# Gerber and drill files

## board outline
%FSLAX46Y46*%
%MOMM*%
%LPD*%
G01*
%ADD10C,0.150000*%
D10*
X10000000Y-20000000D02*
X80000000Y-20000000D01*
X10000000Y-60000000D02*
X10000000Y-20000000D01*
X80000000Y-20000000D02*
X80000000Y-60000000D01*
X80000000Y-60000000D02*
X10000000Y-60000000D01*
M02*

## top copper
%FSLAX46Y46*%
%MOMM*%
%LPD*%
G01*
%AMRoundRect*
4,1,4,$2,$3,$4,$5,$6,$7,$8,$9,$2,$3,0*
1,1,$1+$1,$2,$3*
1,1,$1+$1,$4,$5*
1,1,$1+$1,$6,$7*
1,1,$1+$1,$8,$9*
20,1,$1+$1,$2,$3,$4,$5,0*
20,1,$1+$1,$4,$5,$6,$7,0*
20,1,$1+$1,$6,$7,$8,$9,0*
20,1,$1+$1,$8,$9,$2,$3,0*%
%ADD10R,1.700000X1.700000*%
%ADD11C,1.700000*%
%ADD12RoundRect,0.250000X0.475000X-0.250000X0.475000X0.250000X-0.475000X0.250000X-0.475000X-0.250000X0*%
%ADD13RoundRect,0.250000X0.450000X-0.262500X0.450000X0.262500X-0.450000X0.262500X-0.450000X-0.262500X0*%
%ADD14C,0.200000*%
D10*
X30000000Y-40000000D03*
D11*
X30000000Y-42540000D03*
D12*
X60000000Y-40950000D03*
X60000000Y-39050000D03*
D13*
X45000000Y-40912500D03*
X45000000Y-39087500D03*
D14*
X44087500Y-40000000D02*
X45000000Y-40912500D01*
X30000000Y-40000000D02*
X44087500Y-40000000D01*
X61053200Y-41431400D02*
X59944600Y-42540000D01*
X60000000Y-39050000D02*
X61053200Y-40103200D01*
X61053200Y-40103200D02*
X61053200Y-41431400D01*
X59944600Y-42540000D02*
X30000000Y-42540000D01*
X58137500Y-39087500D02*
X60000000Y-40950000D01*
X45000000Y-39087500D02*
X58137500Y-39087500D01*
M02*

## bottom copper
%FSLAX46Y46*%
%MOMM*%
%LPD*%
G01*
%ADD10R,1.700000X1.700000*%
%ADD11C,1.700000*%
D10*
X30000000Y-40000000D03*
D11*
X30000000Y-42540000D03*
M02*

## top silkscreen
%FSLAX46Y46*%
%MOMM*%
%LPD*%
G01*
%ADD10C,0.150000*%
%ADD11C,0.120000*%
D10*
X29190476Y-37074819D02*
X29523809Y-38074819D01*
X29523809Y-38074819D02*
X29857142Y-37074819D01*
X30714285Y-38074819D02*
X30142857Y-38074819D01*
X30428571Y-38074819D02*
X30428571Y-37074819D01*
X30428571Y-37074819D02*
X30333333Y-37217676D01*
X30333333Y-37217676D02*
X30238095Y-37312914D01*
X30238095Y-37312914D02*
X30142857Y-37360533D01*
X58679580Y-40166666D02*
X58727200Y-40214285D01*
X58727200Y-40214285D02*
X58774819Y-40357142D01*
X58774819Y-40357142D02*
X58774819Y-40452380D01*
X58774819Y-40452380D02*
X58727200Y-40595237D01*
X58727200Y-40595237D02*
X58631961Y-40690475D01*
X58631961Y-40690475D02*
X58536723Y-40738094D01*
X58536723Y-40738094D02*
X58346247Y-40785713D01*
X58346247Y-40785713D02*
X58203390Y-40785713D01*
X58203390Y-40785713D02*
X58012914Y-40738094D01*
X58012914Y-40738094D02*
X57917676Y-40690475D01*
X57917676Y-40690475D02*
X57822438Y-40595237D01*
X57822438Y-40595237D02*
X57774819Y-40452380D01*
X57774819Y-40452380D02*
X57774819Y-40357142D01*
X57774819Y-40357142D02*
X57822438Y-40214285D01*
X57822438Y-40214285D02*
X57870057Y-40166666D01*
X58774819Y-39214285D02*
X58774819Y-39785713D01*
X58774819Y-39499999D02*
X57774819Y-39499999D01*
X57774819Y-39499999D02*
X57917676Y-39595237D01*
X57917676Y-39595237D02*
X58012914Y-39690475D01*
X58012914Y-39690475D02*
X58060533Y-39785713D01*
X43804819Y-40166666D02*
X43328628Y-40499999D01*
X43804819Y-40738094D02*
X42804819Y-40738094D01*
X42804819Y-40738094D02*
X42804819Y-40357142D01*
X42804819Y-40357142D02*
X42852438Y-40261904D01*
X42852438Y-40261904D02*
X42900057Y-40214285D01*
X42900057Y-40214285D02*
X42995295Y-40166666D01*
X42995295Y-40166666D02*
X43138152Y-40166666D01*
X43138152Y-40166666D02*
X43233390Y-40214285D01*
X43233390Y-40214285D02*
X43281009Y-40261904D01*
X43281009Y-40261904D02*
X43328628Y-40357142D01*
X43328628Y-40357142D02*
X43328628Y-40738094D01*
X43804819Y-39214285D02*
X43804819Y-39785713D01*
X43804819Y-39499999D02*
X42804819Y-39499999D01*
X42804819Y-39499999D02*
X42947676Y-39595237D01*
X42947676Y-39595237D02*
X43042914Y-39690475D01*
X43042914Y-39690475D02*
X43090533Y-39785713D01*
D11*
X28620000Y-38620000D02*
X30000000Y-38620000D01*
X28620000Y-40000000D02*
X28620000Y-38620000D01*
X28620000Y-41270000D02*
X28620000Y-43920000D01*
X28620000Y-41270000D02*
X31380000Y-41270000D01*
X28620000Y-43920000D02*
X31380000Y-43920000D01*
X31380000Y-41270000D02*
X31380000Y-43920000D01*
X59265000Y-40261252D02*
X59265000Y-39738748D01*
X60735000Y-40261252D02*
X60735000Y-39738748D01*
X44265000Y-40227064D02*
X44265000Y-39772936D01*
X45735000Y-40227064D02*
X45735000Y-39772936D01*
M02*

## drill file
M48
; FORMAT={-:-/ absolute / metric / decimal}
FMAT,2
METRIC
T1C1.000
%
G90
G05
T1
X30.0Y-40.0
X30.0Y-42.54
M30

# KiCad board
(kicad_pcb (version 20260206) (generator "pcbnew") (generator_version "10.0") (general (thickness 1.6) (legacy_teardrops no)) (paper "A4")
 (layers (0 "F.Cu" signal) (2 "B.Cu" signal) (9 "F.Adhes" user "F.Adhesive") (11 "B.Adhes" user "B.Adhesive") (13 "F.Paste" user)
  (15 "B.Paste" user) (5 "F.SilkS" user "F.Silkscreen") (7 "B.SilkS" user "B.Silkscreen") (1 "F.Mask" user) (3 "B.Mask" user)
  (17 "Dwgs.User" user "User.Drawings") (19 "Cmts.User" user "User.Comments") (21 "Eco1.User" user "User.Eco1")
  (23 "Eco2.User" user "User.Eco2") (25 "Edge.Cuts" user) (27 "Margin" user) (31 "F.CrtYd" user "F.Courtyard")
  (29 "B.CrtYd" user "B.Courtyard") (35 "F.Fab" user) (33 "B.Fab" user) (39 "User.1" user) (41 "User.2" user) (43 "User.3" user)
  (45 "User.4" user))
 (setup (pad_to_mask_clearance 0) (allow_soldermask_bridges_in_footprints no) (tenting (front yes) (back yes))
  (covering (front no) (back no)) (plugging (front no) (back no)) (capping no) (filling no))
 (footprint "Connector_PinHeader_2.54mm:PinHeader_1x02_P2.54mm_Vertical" (layer "F.Cu") (at 30 40)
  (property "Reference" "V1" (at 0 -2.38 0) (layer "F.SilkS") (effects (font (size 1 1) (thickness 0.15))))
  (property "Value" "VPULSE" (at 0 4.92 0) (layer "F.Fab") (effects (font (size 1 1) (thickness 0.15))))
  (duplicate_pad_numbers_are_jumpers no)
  (fp_line (start -1.38 -1.38) (end 0 -1.38) (stroke (width 0.12) (type solid)) (layer "F.SilkS"))
  (fp_line (start -1.38 0) (end -1.38 -1.38) (stroke (width 0.12) (type solid)) (layer "F.SilkS"))
  (fp_line (start -1.38 1.27) (end -1.38 3.92) (stroke (width 0.12) (type solid)) (layer "F.SilkS"))
  (fp_line (start -1.38 1.27) (end 1.38 1.27) (stroke (width 0.12) (type solid)) (layer "F.SilkS"))
  (fp_line (start -1.38 3.92) (end 1.38 3.92) (stroke (width 0.12) (type solid)) (layer "F.SilkS"))
  (fp_line (start 1.38 1.27) (end 1.38 3.92) (stroke (width 0.12) (type solid)) (layer "F.SilkS"))
  (pad "1" thru_hole rect (at 0 0) (size 1.7 1.7) (drill 1) (layers "*.Cu" "*.Mask") (remove_unused_layers no) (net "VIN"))
  (pad "2" thru_hole circle (at 0 2.54) (size 1.7 1.7) (drill 1) (layers "*.Cu" "*.Mask") (remove_unused_layers no) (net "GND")))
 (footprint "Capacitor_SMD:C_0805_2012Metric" (layer "F.Cu") (at 60 40 90)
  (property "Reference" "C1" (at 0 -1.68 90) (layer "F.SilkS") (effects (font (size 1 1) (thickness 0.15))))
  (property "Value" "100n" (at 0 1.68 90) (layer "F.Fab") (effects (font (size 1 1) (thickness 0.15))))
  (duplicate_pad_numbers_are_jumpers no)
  (fp_line (start -0.261252 -0.735) (end 0.261252 -0.735) (stroke (width 0.12) (type solid)) (layer "F.SilkS"))
  (fp_line (start -0.261252 0.735) (end 0.261252 0.735) (stroke (width 0.12) (type solid)) (layer "F.SilkS"))
  (pad "1" smd roundrect (at -0.95 0 90) (size 1 1.45) (layers "F.Cu" "F.Mask" "F.Paste") (roundrect_rratio 0.25) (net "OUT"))
  (pad "2" smd roundrect (at 0.95 0 90) (size 1 1.45) (layers "F.Cu" "F.Mask" "F.Paste") (roundrect_rratio 0.25) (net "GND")))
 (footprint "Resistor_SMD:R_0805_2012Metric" (layer "F.Cu") (at 45 40 90)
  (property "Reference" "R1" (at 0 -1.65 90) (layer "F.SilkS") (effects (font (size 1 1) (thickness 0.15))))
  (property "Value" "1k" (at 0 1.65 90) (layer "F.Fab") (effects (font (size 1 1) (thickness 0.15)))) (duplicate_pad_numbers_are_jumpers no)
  (fp_line (start -0.227064 -0.735) (end 0.227064 -0.735) (stroke (width 0.12) (type solid)) (layer "F.SilkS"))
  (fp_line (start -0.227064 0.735) (end 0.227064 0.735) (stroke (width 0.12) (type solid)) (layer "F.SilkS"))
  (pad "1" smd roundrect (at -0.9125 0 90) (size 1.025 1.4) (layers "F.Cu" "F.Mask" "F.Paste") (roundrect_rratio 0.243902) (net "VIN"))
  (pad "2" smd roundrect (at 0.9125 0 90) (size 1.025 1.4) (layers "F.Cu" "F.Mask" "F.Paste") (roundrect_rratio 0.243902) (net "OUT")))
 (gr_line (start 10 20) (end 80 20) (stroke (width 0.15) (type default)) (layer "Edge.Cuts"))
 (gr_line (start 10 60) (end 10 20) (stroke (width 0.15) (type default)) (layer "Edge.Cuts"))
 (gr_line (start 80 20) (end 80 60) (stroke (width 0.15) (type default)) (layer "Edge.Cuts"))
 (gr_line (start 80 60) (end 10 60) (stroke (width 0.15) (type default)) (layer "Edge.Cuts"))
 (segment (start 44.0875 40) (end 45 40.9125) (width 0.2) (layer "F.Cu") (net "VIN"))
 (segment (start 30 40) (end 44.0875 40) (width 0.2) (layer "F.Cu") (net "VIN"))
 (segment (start 61.0532 41.4314) (end 59.9446 42.54) (width 0.2) (layer "F.Cu") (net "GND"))
 (segment (start 60 39.05) (end 61.0532 40.1032) (width 0.2) (layer "F.Cu") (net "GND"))
 (segment (start 61.0532 40.1032) (end 61.0532 41.4314) (width 0.2) (layer "F.Cu") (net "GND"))
 (segment (start 59.9446 42.54) (end 30 42.54) (width 0.2) (layer "F.Cu") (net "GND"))
 (segment (start 58.1375 39.0875) (end 60 40.95) (width 0.2) (layer "F.Cu") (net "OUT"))
 (segment (start 45 39.0875) (end 58.1375 39.0875) (width 0.2) (layer "F.Cu") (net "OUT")))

